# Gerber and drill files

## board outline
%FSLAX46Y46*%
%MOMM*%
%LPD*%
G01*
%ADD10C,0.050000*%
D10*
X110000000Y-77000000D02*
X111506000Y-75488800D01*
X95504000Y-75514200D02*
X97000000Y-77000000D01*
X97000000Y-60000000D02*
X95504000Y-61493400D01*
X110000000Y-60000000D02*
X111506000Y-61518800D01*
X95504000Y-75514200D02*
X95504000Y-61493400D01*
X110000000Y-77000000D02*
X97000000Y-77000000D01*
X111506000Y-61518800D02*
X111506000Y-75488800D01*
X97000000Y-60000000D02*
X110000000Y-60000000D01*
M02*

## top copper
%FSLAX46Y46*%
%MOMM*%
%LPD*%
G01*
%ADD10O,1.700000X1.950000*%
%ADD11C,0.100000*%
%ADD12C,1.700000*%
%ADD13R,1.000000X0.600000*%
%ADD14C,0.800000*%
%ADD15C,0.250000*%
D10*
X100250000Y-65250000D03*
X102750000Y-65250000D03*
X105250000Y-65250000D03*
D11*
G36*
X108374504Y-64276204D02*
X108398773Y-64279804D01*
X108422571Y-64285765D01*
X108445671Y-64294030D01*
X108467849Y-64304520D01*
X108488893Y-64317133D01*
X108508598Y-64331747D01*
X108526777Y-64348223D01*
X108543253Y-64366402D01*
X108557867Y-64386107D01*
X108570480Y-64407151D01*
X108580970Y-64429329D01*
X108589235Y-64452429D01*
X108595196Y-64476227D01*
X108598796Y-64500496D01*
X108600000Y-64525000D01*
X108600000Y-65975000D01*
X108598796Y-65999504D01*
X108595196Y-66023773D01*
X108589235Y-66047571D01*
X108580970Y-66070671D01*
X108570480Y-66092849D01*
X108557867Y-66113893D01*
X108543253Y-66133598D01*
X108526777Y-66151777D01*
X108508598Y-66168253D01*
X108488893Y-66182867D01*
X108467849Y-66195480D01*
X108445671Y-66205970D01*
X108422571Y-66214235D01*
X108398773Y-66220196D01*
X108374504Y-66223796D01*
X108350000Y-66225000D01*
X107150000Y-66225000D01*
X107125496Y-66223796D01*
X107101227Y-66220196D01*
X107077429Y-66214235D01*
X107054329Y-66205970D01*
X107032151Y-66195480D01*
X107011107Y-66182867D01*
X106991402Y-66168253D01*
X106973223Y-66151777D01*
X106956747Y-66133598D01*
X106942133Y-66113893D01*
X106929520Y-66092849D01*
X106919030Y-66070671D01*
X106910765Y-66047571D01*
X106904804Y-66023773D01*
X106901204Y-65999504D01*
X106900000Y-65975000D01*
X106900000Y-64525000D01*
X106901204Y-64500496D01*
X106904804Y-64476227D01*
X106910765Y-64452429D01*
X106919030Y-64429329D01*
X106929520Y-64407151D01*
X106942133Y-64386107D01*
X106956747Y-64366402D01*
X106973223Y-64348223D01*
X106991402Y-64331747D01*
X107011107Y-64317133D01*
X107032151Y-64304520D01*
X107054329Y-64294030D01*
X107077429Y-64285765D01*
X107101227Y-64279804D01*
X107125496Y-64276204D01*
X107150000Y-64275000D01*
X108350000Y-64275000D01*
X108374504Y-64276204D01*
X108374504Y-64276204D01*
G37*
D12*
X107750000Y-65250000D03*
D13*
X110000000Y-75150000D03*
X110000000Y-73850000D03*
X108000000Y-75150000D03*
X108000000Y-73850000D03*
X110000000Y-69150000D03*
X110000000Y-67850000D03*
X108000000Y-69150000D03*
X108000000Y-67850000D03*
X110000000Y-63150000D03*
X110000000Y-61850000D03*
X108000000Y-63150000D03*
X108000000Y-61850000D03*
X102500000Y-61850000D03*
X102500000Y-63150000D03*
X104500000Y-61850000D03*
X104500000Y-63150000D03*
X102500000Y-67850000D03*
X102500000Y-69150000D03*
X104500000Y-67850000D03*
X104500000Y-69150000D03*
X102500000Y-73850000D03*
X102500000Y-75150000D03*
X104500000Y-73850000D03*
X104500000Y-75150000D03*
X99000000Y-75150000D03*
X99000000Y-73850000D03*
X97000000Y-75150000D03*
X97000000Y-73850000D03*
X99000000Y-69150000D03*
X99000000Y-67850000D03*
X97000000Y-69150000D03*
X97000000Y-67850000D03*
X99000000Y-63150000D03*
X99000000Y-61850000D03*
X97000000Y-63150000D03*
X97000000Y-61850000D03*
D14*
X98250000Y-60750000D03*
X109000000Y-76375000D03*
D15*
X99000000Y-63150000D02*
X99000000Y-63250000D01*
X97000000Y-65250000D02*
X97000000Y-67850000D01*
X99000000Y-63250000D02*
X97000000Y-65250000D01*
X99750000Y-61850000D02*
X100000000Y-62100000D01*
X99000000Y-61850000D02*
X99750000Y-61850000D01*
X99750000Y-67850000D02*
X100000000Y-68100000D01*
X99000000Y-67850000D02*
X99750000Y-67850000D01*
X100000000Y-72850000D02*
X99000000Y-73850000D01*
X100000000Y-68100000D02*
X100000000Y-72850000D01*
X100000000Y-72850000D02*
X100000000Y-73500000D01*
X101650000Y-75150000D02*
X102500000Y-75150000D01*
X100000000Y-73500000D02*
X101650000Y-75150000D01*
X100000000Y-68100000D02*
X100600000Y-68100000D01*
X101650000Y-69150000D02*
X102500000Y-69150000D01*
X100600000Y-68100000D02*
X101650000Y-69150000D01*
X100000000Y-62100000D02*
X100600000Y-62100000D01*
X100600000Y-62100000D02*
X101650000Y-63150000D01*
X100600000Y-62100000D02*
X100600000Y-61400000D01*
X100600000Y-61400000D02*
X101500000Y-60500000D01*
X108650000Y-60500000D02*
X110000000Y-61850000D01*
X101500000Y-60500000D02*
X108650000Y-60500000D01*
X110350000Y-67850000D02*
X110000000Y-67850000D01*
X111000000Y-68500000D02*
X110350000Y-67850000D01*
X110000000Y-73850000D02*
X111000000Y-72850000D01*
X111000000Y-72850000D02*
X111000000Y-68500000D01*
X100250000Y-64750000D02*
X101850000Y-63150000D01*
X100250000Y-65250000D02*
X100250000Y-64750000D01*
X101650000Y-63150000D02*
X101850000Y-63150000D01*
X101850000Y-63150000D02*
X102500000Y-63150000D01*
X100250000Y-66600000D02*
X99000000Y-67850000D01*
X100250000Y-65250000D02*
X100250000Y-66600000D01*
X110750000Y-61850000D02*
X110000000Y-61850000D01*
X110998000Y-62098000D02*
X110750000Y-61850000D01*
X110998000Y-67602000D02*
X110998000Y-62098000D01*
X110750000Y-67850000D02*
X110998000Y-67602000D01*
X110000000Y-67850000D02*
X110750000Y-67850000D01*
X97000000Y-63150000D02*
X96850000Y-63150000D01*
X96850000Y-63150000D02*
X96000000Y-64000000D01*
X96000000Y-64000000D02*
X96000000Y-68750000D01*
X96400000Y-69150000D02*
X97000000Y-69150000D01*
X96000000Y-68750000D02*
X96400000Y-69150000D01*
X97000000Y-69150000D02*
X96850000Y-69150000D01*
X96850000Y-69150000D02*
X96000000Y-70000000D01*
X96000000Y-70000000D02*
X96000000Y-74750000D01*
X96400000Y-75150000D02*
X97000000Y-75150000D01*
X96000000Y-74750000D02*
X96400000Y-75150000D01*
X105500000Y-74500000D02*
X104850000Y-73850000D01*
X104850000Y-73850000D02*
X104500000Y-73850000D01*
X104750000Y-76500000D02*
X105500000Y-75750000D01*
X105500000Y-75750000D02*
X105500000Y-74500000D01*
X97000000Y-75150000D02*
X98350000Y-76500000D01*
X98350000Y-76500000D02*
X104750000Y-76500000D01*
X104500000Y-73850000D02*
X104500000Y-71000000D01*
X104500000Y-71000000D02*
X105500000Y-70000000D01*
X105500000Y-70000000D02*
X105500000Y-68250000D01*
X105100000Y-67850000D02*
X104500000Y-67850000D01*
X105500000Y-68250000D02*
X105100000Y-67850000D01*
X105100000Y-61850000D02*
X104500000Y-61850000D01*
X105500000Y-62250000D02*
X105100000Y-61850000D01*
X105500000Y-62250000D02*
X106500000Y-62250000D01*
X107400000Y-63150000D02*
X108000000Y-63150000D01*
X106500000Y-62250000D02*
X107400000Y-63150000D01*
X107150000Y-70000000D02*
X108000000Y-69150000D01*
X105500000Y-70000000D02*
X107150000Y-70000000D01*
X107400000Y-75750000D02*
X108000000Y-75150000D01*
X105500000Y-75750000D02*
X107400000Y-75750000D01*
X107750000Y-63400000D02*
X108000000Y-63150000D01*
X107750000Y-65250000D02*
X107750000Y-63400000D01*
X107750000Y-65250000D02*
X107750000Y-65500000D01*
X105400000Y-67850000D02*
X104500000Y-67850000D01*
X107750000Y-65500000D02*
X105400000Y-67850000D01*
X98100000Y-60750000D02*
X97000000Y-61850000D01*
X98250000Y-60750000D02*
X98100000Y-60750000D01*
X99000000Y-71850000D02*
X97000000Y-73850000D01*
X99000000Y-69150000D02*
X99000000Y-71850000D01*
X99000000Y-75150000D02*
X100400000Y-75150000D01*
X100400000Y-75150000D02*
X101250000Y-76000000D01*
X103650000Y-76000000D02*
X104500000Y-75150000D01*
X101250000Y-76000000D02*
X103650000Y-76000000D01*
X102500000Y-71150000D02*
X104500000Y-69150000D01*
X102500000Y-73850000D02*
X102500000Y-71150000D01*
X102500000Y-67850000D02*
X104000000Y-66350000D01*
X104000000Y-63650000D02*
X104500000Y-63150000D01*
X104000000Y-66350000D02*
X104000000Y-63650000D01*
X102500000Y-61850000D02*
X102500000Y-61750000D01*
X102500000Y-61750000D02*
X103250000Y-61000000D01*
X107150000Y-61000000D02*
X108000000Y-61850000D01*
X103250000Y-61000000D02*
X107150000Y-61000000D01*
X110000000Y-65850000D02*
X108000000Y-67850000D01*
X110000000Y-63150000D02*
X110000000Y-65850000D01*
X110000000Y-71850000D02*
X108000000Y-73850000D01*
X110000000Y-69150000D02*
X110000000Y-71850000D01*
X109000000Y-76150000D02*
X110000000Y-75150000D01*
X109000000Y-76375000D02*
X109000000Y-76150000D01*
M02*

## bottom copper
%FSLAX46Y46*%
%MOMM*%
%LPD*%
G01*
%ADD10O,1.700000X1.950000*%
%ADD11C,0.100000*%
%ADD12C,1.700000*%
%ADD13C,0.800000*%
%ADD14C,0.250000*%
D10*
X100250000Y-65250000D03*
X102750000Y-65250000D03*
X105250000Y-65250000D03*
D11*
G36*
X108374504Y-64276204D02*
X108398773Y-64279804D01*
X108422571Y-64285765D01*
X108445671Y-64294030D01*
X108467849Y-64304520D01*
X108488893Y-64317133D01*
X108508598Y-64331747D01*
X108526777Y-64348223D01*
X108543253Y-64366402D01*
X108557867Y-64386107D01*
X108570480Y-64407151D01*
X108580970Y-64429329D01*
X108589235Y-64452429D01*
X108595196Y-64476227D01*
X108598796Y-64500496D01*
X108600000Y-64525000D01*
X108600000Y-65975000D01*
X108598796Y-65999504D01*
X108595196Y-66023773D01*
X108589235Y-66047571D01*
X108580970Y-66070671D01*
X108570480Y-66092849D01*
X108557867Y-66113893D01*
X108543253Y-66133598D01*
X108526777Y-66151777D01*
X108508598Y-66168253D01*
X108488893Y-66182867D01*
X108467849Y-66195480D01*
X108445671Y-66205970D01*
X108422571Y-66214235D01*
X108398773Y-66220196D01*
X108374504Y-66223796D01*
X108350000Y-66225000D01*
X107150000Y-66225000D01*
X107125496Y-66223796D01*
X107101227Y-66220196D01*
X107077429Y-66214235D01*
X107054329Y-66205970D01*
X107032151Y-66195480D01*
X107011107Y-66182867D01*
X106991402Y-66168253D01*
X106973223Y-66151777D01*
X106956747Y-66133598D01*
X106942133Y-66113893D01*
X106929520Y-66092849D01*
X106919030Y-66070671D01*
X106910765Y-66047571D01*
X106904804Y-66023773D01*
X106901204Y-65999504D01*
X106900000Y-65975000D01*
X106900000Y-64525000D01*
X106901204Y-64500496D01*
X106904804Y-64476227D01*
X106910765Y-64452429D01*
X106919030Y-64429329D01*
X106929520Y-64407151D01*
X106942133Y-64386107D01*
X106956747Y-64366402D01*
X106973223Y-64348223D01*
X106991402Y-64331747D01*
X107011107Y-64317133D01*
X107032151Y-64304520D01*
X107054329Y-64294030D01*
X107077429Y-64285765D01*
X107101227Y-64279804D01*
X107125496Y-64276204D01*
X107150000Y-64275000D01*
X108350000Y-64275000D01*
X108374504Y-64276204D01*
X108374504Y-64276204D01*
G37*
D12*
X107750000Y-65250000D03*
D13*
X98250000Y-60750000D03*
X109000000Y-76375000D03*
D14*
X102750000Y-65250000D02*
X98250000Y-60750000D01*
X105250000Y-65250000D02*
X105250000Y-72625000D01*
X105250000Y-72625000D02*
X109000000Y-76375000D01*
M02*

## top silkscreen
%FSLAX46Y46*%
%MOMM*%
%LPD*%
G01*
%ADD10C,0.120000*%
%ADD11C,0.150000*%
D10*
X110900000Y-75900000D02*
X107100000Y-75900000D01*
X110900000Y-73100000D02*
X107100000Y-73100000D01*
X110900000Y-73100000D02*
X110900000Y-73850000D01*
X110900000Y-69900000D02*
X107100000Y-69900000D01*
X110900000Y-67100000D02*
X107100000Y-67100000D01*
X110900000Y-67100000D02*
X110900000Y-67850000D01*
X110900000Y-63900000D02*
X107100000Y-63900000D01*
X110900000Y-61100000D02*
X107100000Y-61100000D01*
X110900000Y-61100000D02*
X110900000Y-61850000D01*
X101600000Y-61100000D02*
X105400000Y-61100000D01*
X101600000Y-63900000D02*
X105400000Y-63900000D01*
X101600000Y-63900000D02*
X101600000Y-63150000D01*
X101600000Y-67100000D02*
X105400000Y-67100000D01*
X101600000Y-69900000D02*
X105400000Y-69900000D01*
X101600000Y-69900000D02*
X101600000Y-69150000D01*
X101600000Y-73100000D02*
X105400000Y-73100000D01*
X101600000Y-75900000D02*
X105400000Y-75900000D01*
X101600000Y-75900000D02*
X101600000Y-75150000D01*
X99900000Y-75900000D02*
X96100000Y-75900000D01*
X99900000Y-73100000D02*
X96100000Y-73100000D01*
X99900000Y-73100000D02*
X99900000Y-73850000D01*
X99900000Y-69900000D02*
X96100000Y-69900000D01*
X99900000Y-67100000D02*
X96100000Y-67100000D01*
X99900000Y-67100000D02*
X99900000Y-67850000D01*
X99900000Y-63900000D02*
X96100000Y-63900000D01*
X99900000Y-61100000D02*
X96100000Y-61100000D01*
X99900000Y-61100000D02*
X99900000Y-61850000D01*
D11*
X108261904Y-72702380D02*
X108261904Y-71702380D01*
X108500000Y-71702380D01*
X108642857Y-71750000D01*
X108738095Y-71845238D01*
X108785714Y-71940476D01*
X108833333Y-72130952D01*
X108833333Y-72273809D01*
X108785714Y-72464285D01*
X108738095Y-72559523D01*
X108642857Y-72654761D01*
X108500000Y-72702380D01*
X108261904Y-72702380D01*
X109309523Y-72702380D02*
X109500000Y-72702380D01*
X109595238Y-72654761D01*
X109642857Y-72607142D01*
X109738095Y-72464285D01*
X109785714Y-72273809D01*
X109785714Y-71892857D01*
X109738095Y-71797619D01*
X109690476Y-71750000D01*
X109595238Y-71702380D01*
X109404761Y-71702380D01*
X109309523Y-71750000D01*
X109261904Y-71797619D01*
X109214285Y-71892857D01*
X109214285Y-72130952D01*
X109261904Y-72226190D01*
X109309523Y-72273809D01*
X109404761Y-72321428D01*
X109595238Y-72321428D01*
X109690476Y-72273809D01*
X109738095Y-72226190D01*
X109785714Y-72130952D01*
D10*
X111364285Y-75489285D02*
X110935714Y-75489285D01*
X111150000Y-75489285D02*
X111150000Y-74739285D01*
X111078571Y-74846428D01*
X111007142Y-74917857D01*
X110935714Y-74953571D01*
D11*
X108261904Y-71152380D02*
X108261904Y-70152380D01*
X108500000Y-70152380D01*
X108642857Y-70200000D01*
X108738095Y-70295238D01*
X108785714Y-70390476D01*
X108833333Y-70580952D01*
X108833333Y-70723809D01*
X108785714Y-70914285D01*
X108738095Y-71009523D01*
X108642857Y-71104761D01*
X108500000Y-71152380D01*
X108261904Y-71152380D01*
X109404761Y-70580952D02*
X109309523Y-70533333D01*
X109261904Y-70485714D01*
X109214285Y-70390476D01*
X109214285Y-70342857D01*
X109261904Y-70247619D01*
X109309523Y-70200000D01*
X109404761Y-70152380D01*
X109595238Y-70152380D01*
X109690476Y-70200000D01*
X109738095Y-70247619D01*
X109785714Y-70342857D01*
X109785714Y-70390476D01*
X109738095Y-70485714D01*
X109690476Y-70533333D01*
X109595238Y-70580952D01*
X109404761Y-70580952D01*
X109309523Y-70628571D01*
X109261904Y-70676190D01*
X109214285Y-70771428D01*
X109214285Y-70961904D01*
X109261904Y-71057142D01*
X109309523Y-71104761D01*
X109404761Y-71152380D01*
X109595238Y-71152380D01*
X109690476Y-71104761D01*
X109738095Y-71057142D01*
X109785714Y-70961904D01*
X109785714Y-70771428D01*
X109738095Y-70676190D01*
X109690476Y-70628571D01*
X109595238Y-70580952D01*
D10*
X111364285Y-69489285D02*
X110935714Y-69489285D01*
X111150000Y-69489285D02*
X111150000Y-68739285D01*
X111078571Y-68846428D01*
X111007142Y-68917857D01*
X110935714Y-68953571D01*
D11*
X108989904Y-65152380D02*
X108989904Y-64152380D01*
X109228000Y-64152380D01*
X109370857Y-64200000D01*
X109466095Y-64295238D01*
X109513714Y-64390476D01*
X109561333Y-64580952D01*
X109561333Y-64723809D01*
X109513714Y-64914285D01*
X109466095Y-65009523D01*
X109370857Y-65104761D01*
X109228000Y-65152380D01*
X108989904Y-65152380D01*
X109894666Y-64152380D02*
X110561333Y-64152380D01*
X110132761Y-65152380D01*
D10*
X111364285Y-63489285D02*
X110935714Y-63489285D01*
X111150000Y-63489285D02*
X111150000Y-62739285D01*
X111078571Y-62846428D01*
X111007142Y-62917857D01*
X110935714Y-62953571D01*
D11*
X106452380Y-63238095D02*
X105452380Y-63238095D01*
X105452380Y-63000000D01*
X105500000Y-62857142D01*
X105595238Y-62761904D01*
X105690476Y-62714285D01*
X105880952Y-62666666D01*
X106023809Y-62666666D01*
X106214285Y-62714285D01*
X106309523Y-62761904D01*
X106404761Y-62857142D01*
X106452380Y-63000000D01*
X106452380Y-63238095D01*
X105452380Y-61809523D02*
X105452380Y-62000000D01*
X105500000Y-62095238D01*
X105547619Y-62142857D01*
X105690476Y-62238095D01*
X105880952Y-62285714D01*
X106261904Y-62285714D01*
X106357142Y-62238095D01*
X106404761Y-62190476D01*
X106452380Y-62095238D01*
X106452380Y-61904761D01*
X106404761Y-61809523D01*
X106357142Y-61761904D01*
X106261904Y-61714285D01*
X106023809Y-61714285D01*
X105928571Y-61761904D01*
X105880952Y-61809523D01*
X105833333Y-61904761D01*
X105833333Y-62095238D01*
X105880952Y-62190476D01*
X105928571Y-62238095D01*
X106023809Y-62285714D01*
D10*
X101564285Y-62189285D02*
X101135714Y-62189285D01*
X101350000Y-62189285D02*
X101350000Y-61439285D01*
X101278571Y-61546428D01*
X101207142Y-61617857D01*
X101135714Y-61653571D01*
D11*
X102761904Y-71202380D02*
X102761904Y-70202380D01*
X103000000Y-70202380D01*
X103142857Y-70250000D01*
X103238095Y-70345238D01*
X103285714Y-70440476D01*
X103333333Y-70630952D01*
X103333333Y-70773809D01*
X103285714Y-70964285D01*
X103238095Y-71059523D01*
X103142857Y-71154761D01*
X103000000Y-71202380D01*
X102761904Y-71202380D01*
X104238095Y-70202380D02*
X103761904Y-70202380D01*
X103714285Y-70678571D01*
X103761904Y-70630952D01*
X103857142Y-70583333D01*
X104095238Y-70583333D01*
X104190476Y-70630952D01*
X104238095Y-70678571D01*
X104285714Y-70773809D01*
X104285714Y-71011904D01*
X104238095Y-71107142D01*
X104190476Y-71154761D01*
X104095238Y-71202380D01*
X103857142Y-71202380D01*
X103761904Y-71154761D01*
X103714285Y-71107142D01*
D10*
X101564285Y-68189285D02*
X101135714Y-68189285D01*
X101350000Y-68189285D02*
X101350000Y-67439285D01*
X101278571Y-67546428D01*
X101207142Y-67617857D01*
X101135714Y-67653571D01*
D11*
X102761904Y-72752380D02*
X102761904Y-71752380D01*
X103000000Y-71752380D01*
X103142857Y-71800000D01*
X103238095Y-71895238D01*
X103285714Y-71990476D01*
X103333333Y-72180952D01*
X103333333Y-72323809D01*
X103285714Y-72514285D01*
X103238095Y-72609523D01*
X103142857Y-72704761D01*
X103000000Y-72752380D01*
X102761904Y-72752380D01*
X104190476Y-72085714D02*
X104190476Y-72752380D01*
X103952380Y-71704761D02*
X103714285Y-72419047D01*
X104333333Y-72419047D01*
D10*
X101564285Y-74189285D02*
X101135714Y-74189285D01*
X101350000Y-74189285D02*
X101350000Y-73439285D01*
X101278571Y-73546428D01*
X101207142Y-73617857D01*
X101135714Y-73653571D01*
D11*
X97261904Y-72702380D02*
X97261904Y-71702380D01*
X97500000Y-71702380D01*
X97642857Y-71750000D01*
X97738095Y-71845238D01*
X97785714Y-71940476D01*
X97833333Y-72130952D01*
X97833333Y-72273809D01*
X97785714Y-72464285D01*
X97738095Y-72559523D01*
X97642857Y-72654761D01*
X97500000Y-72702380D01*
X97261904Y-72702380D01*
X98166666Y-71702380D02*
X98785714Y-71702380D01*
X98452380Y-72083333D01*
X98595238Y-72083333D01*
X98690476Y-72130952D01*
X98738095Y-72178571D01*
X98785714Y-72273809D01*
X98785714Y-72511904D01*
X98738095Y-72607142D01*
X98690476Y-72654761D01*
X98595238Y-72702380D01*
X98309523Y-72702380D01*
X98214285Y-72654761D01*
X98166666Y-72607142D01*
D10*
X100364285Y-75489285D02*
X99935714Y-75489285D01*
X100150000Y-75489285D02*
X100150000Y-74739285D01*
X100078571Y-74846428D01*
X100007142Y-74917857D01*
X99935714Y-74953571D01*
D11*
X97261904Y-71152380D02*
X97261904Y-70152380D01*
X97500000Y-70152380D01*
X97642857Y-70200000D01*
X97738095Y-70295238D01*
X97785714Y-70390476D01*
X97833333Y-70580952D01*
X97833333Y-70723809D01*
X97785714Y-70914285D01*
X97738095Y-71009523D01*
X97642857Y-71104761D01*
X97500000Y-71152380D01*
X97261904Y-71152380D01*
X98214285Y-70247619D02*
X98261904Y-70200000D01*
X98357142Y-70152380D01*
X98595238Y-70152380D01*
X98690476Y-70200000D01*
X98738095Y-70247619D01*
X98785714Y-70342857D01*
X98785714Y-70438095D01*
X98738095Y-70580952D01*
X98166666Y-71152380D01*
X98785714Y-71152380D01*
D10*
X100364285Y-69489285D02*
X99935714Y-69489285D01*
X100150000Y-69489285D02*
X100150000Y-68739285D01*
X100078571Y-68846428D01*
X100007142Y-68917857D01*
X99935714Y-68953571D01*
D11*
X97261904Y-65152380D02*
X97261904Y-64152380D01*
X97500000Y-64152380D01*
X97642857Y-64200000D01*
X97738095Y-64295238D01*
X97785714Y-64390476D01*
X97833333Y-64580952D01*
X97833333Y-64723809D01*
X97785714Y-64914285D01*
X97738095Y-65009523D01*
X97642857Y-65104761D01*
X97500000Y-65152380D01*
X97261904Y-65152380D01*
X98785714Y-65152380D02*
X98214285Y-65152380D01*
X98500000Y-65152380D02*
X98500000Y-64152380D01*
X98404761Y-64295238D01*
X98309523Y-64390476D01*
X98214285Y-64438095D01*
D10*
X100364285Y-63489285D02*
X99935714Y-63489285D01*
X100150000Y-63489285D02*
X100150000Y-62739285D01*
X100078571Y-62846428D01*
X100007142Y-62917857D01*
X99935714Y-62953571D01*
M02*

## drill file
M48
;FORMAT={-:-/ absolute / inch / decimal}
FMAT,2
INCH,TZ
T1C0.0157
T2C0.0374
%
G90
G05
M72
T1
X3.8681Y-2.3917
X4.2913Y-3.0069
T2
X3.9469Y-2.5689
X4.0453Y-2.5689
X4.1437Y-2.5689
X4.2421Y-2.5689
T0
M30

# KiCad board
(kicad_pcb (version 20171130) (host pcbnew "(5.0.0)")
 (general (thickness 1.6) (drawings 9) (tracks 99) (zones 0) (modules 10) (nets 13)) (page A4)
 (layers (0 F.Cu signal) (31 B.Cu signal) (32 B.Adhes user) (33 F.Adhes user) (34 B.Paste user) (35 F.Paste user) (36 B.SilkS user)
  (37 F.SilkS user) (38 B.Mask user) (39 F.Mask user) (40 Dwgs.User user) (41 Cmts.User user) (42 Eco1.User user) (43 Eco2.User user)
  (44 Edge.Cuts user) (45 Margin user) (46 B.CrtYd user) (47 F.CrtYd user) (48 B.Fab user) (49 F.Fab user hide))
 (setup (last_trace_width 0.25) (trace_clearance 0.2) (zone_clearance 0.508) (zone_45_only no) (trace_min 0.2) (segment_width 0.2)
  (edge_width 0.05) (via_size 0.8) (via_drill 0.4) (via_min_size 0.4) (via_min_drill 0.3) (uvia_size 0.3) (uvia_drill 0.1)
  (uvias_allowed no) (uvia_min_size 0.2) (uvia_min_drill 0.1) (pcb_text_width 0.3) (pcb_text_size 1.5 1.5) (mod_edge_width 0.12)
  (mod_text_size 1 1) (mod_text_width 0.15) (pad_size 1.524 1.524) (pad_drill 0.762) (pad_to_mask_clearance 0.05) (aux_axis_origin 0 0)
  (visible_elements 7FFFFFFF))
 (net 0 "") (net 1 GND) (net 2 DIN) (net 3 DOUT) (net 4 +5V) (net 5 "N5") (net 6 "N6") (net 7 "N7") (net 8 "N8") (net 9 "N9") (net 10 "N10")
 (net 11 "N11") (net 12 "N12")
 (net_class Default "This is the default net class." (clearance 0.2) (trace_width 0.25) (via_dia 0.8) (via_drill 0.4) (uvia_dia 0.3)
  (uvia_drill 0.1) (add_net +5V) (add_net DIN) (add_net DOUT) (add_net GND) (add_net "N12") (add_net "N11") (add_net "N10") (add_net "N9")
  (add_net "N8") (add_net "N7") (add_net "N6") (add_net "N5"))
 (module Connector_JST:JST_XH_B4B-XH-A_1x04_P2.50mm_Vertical (layer B.Cu) (at 107.75 65.25 180)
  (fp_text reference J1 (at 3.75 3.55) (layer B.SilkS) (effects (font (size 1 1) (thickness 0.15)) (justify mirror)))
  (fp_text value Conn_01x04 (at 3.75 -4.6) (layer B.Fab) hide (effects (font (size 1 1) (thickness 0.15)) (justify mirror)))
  (pad 4 thru_hole oval (at 7.5 0 180) (size 1.7 1.95) (drill 0.95) (layers *.Cu *.Mask) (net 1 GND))
  (pad 3 thru_hole oval (at 5 0 180) (size 1.7 1.95) (drill 0.95) (layers *.Cu *.Mask) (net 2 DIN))
  (pad 2 thru_hole oval (at 2.5 0 180) (size 1.7 1.95) (drill 0.95) (layers *.Cu *.Mask) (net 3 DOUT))
  (pad 1 thru_hole roundrect (at 0 0 180) (size 1.7 1.95) (drill 0.95) (layers *.Cu *.Mask) (roundrect_rratio 0.147059) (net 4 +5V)))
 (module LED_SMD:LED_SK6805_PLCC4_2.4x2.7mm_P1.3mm (layer F.Cu) (at 109 74.5 180)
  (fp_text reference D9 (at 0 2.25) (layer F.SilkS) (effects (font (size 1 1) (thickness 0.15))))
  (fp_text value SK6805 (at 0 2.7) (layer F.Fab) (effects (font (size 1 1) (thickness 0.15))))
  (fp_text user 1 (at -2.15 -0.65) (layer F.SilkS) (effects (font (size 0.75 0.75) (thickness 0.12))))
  (fp_line (start -1.9 -1.4) (end 1.9 -1.4) (layer F.SilkS) (width 0.12))
  (fp_line (start -1.9 1.4) (end 1.9 1.4) (layer F.SilkS) (width 0.12))
  (fp_line (start -1.9 1.4) (end -1.9 0.65) (layer F.SilkS) (width 0.12))
  (pad 1 smd rect (at -1 -0.65 180) (size 1 0.6) (layers F.Cu F.Paste F.Mask) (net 3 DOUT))
  (pad 2 smd rect (at -1 0.65 180) (size 1 0.6) (layers F.Cu F.Paste F.Mask) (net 1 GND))
  (pad 4 smd rect (at 1 -0.65 180) (size 1 0.6) (layers F.Cu F.Paste F.Mask) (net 4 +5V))
  (pad 3 smd rect (at 1 0.65 180) (size 1 0.6) (layers F.Cu F.Paste F.Mask) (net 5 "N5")))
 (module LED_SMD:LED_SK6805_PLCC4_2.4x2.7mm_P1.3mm (layer F.Cu) (at 109 68.5 180)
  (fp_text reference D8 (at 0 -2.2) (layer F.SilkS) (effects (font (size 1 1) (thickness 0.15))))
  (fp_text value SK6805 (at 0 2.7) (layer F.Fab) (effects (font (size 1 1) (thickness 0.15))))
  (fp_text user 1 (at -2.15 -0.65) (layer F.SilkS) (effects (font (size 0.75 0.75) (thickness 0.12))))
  (fp_line (start -1.9 -1.4) (end 1.9 -1.4) (layer F.SilkS) (width 0.12))
  (fp_line (start -1.9 1.4) (end 1.9 1.4) (layer F.SilkS) (width 0.12))
  (fp_line (start -1.9 1.4) (end -1.9 0.65) (layer F.SilkS) (width 0.12))
  (pad 1 smd rect (at -1 -0.65 180) (size 1 0.6) (layers F.Cu F.Paste F.Mask) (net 5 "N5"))
  (pad 2 smd rect (at -1 0.65 180) (size 1 0.6) (layers F.Cu F.Paste F.Mask) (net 1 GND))
  (pad 4 smd rect (at 1 -0.65 180) (size 1 0.6) (layers F.Cu F.Paste F.Mask) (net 4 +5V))
  (pad 3 smd rect (at 1 0.65 180) (size 1 0.6) (layers F.Cu F.Paste F.Mask) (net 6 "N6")))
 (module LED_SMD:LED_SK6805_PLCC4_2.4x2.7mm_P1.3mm (layer F.Cu) (at 109 62.5 180)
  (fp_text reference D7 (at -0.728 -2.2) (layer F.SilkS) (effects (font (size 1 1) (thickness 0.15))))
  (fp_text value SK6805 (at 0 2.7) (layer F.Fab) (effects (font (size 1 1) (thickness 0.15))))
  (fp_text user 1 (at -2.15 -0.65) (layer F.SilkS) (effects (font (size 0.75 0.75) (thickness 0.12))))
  (fp_line (start -1.9 -1.4) (end 1.9 -1.4) (layer F.SilkS) (width 0.12))
  (fp_line (start -1.9 1.4) (end 1.9 1.4) (layer F.SilkS) (width 0.12))
  (fp_line (start -1.9 1.4) (end -1.9 0.65) (layer F.SilkS) (width 0.12))
  (pad 1 smd rect (at -1 -0.65 180) (size 1 0.6) (layers F.Cu F.Paste F.Mask) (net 6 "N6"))
  (pad 2 smd rect (at -1 0.65 180) (size 1 0.6) (layers F.Cu F.Paste F.Mask) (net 1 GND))
  (pad 4 smd rect (at 1 -0.65 180) (size 1 0.6) (layers F.Cu F.Paste F.Mask) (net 4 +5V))
  (pad 3 smd rect (at 1 0.65 180) (size 1 0.6) (layers F.Cu F.Paste F.Mask) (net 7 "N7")))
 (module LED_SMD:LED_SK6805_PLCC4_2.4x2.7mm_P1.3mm (layer F.Cu) (at 103.5 62.5)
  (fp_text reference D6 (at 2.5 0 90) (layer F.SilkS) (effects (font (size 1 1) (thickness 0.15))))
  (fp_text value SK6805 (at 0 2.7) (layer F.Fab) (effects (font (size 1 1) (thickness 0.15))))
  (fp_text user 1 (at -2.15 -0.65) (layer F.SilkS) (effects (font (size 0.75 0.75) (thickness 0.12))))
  (fp_line (start -1.9 -1.4) (end 1.9 -1.4) (layer F.SilkS) (width 0.12))
  (fp_line (start -1.9 1.4) (end 1.9 1.4) (layer F.SilkS) (width 0.12))
  (fp_line (start -1.9 1.4) (end -1.9 0.65) (layer F.SilkS) (width 0.12))
  (pad 1 smd rect (at -1 -0.65) (size 1 0.6) (layers F.Cu F.Paste F.Mask) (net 7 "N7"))
  (pad 2 smd rect (at -1 0.65) (size 1 0.6) (layers F.Cu F.Paste F.Mask) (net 1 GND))
  (pad 4 smd rect (at 1 -0.65) (size 1 0.6) (layers F.Cu F.Paste F.Mask) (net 4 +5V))
  (pad 3 smd rect (at 1 0.65) (size 1 0.6) (layers F.Cu F.Paste F.Mask) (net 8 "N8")))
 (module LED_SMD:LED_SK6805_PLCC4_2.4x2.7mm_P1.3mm (layer F.Cu) (at 103.5 68.5)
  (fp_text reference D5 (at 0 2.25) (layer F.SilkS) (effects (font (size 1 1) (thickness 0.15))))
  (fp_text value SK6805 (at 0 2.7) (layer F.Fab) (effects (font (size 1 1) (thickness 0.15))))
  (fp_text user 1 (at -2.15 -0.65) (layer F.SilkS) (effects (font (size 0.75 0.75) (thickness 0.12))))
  (fp_line (start -1.9 -1.4) (end 1.9 -1.4) (layer F.SilkS) (width 0.12))
  (fp_line (start -1.9 1.4) (end 1.9 1.4) (layer F.SilkS) (width 0.12))
  (fp_line (start -1.9 1.4) (end -1.9 0.65) (layer F.SilkS) (width 0.12))
  (pad 1 smd rect (at -1 -0.65) (size 1 0.6) (layers F.Cu F.Paste F.Mask) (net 8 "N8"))
  (pad 2 smd rect (at -1 0.65) (size 1 0.6) (layers F.Cu F.Paste F.Mask) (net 1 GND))
  (pad 4 smd rect (at 1 -0.65) (size 1 0.6) (layers F.Cu F.Paste F.Mask) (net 4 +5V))
  (pad 3 smd rect (at 1 0.65) (size 1 0.6) (layers F.Cu F.Paste F.Mask) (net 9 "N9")))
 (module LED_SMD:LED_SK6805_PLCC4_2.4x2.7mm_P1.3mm (layer F.Cu) (at 103.5 74.5)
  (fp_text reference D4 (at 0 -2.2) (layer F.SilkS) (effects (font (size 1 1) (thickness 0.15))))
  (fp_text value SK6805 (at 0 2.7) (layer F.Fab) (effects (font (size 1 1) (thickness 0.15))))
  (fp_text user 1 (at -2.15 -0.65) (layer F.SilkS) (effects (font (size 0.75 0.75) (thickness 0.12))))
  (fp_line (start -1.9 -1.4) (end 1.9 -1.4) (layer F.SilkS) (width 0.12))
  (fp_line (start -1.9 1.4) (end 1.9 1.4) (layer F.SilkS) (width 0.12))
  (fp_line (start -1.9 1.4) (end -1.9 0.65) (layer F.SilkS) (width 0.12))
  (pad 1 smd rect (at -1 -0.65) (size 1 0.6) (layers F.Cu F.Paste F.Mask) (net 9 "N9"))
  (pad 2 smd rect (at -1 0.65) (size 1 0.6) (layers F.Cu F.Paste F.Mask) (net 1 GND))
  (pad 4 smd rect (at 1 -0.65) (size 1 0.6) (layers F.Cu F.Paste F.Mask) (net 4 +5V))
  (pad 3 smd rect (at 1 0.65) (size 1 0.6) (layers F.Cu F.Paste F.Mask) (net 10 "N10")))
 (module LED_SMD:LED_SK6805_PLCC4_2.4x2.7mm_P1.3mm (layer F.Cu) (at 98 74.5 180)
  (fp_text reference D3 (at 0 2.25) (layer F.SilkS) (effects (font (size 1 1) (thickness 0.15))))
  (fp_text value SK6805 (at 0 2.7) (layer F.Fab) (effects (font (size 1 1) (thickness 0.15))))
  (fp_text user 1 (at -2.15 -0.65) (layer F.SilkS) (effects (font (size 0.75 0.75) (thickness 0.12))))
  (fp_line (start -1.9 -1.4) (end 1.9 -1.4) (layer F.SilkS) (width 0.12))
  (fp_line (start -1.9 1.4) (end 1.9 1.4) (layer F.SilkS) (width 0.12))
  (fp_line (start -1.9 1.4) (end -1.9 0.65) (layer F.SilkS) (width 0.12))
  (pad 1 smd rect (at -1 -0.65 180) (size 1 0.6) (layers F.Cu F.Paste F.Mask) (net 10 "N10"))
  (pad 2 smd rect (at -1 0.65 180) (size 1 0.6) (layers F.Cu F.Paste F.Mask) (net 1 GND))
  (pad 4 smd rect (at 1 -0.65 180) (size 1 0.6) (layers F.Cu F.Paste F.Mask) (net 4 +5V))
  (pad 3 smd rect (at 1 0.65 180) (size 1 0.6) (layers F.Cu F.Paste F.Mask) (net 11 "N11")))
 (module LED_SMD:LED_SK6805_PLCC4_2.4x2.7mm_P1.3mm (layer F.Cu) (at 98 68.5 180)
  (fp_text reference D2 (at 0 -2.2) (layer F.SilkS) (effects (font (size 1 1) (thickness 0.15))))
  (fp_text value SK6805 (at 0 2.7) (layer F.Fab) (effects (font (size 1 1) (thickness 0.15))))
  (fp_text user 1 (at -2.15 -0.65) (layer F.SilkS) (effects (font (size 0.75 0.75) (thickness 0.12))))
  (fp_line (start -1.9 -1.4) (end 1.9 -1.4) (layer F.SilkS) (width 0.12))
  (fp_line (start -1.9 1.4) (end 1.9 1.4) (layer F.SilkS) (width 0.12))
  (fp_line (start -1.9 1.4) (end -1.9 0.65) (layer F.SilkS) (width 0.12))
  (pad 1 smd rect (at -1 -0.65 180) (size 1 0.6) (layers F.Cu F.Paste F.Mask) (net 11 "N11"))
  (pad 2 smd rect (at -1 0.65 180) (size 1 0.6) (layers F.Cu F.Paste F.Mask) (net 1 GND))
  (pad 4 smd rect (at 1 -0.65 180) (size 1 0.6) (layers F.Cu F.Paste F.Mask) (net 4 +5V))
  (pad 3 smd rect (at 1 0.65 180) (size 1 0.6) (layers F.Cu F.Paste F.Mask) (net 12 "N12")))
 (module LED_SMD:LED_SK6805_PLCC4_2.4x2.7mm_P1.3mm (layer F.Cu) (at 98 62.5 180)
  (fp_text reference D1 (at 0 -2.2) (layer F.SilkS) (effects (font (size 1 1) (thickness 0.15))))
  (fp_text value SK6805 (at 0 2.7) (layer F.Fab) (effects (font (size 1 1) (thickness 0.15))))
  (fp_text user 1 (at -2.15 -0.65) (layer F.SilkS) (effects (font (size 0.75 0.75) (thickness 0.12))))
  (fp_line (start -1.9 -1.4) (end 1.9 -1.4) (layer F.SilkS) (width 0.12))
  (fp_line (start -1.9 1.4) (end 1.9 1.4) (layer F.SilkS) (width 0.12))
  (fp_line (start -1.9 1.4) (end -1.9 0.65) (layer F.SilkS) (width 0.12))
  (pad 1 smd rect (at -1 -0.65 180) (size 1 0.6) (layers F.Cu F.Paste F.Mask) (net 12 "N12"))
  (pad 2 smd rect (at -1 0.65 180) (size 1 0.6) (layers F.Cu F.Paste F.Mask) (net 1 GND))
  (pad 4 smd rect (at 1 -0.65 180) (size 1 0.6) (layers F.Cu F.Paste F.Mask) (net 4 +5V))
  (pad 3 smd rect (at 1 0.65 180) (size 1 0.6) (layers F.Cu F.Paste F.Mask) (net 2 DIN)))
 (gr_line (start 110 77) (end 111.506 75.4888) (layer Edge.Cuts) (width 0.05))
 (gr_line (start 95.504 75.5142) (end 97 77) (layer Edge.Cuts) (width 0.05))
 (gr_line (start 97 60) (end 95.504 61.4934) (layer Edge.Cuts) (width 0.05))
 (gr_line (start 110 60) (end 111.506 61.5188) (layer Edge.Cuts) (width 0.05))
 (gr_line (start 95.504 75.5142) (end 95.504 61.4934) (layer Edge.Cuts) (width 0.05))
 (gr_line (start 110 77) (end 97 77) (layer Edge.Cuts) (width 0.05))
 (gr_line (start 111.506 61.5188) (end 111.506 75.4888) (layer Edge.Cuts) (width 0.05))
 (gr_line (start 97 60) (end 110 60) (layer Edge.Cuts) (width 0.05))
 (segment (start 99 63.15) (end 99 63.25) (width 0.25) (layer F.Cu) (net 12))
 (segment (start 97 65.25) (end 97 67.85) (width 0.25) (layer F.Cu) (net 12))
 (segment (start 99 63.25) (end 97 65.25) (width 0.25) (layer F.Cu) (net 12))
 (segment (start 99.75 61.85) (end 100 62.1) (width 0.25) (layer F.Cu) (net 1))
 (segment (start 99 61.85) (end 99.75 61.85) (width 0.25) (layer F.Cu) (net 1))
 (segment (start 99.75 67.85) (end 100 68.1) (width 0.25) (layer F.Cu) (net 1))
 (segment (start 99 67.85) (end 99.75 67.85) (width 0.25) (layer F.Cu) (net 1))
 (segment (start 100 72.85) (end 99 73.85) (width 0.25) (layer F.Cu) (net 1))
 (segment (start 100 68.1) (end 100 72.85) (width 0.25) (layer F.Cu) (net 1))
 (segment (start 100 72.85) (end 100 73.5) (width 0.25) (layer F.Cu) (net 1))
 (segment (start 101.65 75.15) (end 102.5 75.15) (width 0.25) (layer F.Cu) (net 1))
 (segment (start 100 73.5) (end 101.65 75.15) (width 0.25) (layer F.Cu) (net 1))
 (segment (start 100 68.1) (end 100.6 68.1) (width 0.25) (layer F.Cu) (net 1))
 (segment (start 101.65 69.15) (end 102.5 69.15) (width 0.25) (layer F.Cu) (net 1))
 (segment (start 100.6 68.1) (end 101.65 69.15) (width 0.25) (layer F.Cu) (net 1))
 (segment (start 100 62.1) (end 100.6 62.1) (width 0.25) (layer F.Cu) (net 1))
 (segment (start 100.6 62.1) (end 101.65 63.15) (width 0.25) (layer F.Cu) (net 1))
 (segment (start 100.6 62.1) (end 100.6 61.4) (width 0.25) (layer F.Cu) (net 1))
 (segment (start 100.6 61.4) (end 101.5 60.5) (width 0.25) (layer F.Cu) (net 1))
 (segment (start 108.65 60.5) (end 110 61.85) (width 0.25) (layer F.Cu) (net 1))
 (segment (start 101.5 60.5) (end 108.65 60.5) (width 0.25) (layer F.Cu) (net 1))
 (segment (start 110.35 67.85) (end 110 67.85) (width 0.25) (layer F.Cu) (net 1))
 (segment (start 111 68.5) (end 110.35 67.85) (width 0.25) (layer F.Cu) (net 1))
 (segment (start 110 73.85) (end 111 72.85) (width 0.25) (layer F.Cu) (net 1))
 (segment (start 111 72.85) (end 111 68.5) (width 0.25) (layer F.Cu) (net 1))
 (segment (start 100.25 64.75) (end 101.85 63.15) (width 0.25) (layer F.Cu) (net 1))
 (segment (start 100.25 65.25) (end 100.25 64.75) (width 0.25) (layer F.Cu) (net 1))
 (segment (start 101.65 63.15) (end 101.85 63.15) (width 0.25) (layer F.Cu) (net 1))
 (segment (start 101.85 63.15) (end 102.5 63.15) (width 0.25) (layer F.Cu) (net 1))
 (segment (start 100.25 66.6) (end 99 67.85) (width 0.25) (layer F.Cu) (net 1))
 (segment (start 100.25 65.25) (end 100.25 66.6) (width 0.25) (layer F.Cu) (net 1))
 (segment (start 110.75 61.85) (end 110 61.85) (width 0.25) (layer F.Cu) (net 1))
 (segment (start 110.998 62.098) (end 110.75 61.85) (width 0.25) (layer F.Cu) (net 1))
 (segment (start 110.998 67.602) (end 110.998 62.098) (width 0.25) (layer F.Cu) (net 1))
 (segment (start 110.75 67.85) (end 110.998 67.602) (width 0.25) (layer F.Cu) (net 1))
 (segment (start 110 67.85) (end 110.75 67.85) (width 0.25) (layer F.Cu) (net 1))
 (segment (start 97 63.15) (end 96.85 63.15) (width 0.25) (layer F.Cu) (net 4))
 (segment (start 96.85 63.15) (end 96 64) (width 0.25) (layer F.Cu) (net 4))
 (segment (start 96 64) (end 96 68.75) (width 0.25) (layer F.Cu) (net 4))
 (segment (start 96.4 69.15) (end 97 69.15) (width 0.25) (layer F.Cu) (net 4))
 (segment (start 96 68.75) (end 96.4 69.15) (width 0.25) (layer F.Cu) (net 4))
 (segment (start 97 69.15) (end 96.85 69.15) (width 0.25) (layer F.Cu) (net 4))
 (segment (start 96.85 69.15) (end 96 70) (width 0.25) (layer F.Cu) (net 4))
 (segment (start 96 70) (end 96 74.75) (width 0.25) (layer F.Cu) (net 4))
 (segment (start 96.4 75.15) (end 97 75.15) (width 0.25) (layer F.Cu) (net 4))
 (segment (start 96 74.75) (end 96.4 75.15) (width 0.25) (layer F.Cu) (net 4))
 (segment (start 105.5 74.5) (end 104.85 73.85) (width 0.25) (layer F.Cu) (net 4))
 (segment (start 104.85 73.85) (end 104.5 73.85) (width 0.25) (layer F.Cu) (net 4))
 (segment (start 104.75 76.5) (end 105.5 75.75) (width 0.25) (layer F.Cu) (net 4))
 (segment (start 105.5 75.75) (end 105.5 74.5) (width 0.25) (layer F.Cu) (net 4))
 (segment (start 97 75.15) (end 98.35 76.5) (width 0.25) (layer F.Cu) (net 4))
 (segment (start 98.35 76.5) (end 104.75 76.5) (width 0.25) (layer F.Cu) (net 4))
 (segment (start 104.5 73.85) (end 104.5 71) (width 0.25) (layer F.Cu) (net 4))
 (segment (start 104.5 71) (end 105.5 70) (width 0.25) (layer F.Cu) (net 4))
 (segment (start 105.5 70) (end 105.5 68.25) (width 0.25) (layer F.Cu) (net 4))
 (segment (start 105.1 67.85) (end 104.5 67.85) (width 0.25) (layer F.Cu) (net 4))
 (segment (start 105.5 68.25) (end 105.1 67.85) (width 0.25) (layer F.Cu) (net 4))
 (segment (start 105.1 61.85) (end 104.5 61.85) (width 0.25) (layer F.Cu) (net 4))
 (segment (start 105.5 62.25) (end 105.1 61.85) (width 0.25) (layer F.Cu) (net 4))
 (segment (start 105.5 62.25) (end 106.5 62.25) (width 0.25) (layer F.Cu) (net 4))
 (segment (start 107.4 63.15) (end 108 63.15) (width 0.25) (layer F.Cu) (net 4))
 (segment (start 106.5 62.25) (end 107.4 63.15) (width 0.25) (layer F.Cu) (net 4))
 (segment (start 107.15 70) (end 108 69.15) (width 0.25) (layer F.Cu) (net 4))
 (segment (start 105.5 70) (end 107.15 70) (width 0.25) (layer F.Cu) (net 4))
 (segment (start 107.4 75.75) (end 108 75.15) (width 0.25) (layer F.Cu) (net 4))
 (segment (start 105.5 75.75) (end 107.4 75.75) (width 0.25) (layer F.Cu) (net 4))
 (segment (start 107.75 63.4) (end 108 63.15) (width 0.25) (layer F.Cu) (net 4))
 (segment (start 107.75 65.25) (end 107.75 63.4) (width 0.25) (layer F.Cu) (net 4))
 (segment (start 107.75 65.25) (end 107.75 65.5) (width 0.25) (layer F.Cu) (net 4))
 (segment (start 105.4 67.85) (end 104.5 67.85) (width 0.25) (layer F.Cu) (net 4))
 (segment (start 107.75 65.5) (end 105.4 67.85) (width 0.25) (layer F.Cu) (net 4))
 (via (at 98.25 60.75) (size 0.8) (drill 0.4) (layers F.Cu B.Cu) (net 2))
 (segment (start 102.75 65.25) (end 98.25 60.75) (width 0.25) (layer B.Cu) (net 2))
 (segment (start 98.1 60.75) (end 97 61.85) (width 0.25) (layer F.Cu) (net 2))
 (segment (start 98.25 60.75) (end 98.1 60.75) (width 0.25) (layer F.Cu) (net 2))
 (segment (start 99 71.85) (end 97 73.85) (width 0.25) (layer F.Cu) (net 11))
 (segment (start 99 69.15) (end 99 71.85) (width 0.25) (layer F.Cu) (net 11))
 (segment (start 99 75.15) (end 100.4 75.15) (width 0.25) (layer F.Cu) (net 10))
 (segment (start 100.4 75.15) (end 101.25 76) (width 0.25) (layer F.Cu) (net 10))
 (segment (start 103.65 76) (end 104.5 75.15) (width 0.25) (layer F.Cu) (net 10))
 (segment (start 101.25 76) (end 103.65 76) (width 0.25) (layer F.Cu) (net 10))
 (segment (start 102.5 71.15) (end 104.5 69.15) (width 0.25) (layer F.Cu) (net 9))
 (segment (start 102.5 73.85) (end 102.5 71.15) (width 0.25) (layer F.Cu) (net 9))
 (segment (start 102.5 67.85) (end 104 66.35) (width 0.25) (layer F.Cu) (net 8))
 (segment (start 104 63.65) (end 104.5 63.15) (width 0.25) (layer F.Cu) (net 8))
 (segment (start 104 66.35) (end 104 63.65) (width 0.25) (layer F.Cu) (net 8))
 (segment (start 102.5 61.85) (end 102.5 61.75) (width 0.25) (layer F.Cu) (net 7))
 (segment (start 102.5 61.75) (end 103.25 61) (width 0.25) (layer F.Cu) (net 7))
 (segment (start 107.15 61) (end 108 61.85) (width 0.25) (layer F.Cu) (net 7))
 (segment (start 103.25 61) (end 107.15 61) (width 0.25) (layer F.Cu) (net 7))
 (segment (start 110 65.85) (end 108 67.85) (width 0.25) (layer F.Cu) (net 6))
 (segment (start 110 63.15) (end 110 65.85) (width 0.25) (layer F.Cu) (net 6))
 (segment (start 110 71.85) (end 108 73.85) (width 0.25) (layer F.Cu) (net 5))
 (segment (start 110 69.15) (end 110 71.85) (width 0.25) (layer F.Cu) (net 5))
 (via (at 109 76.375) (size 0.8) (drill 0.4) (layers F.Cu B.Cu) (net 3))
 (segment (start 105.25 65.25) (end 105.25 72.625) (width 0.25) (layer B.Cu) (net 3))
 (segment (start 105.25 72.625) (end 109 76.375) (width 0.25) (layer B.Cu) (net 3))
 (segment (start 109 76.15) (end 110 75.15) (width 0.25) (layer F.Cu) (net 3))
 (segment (start 109 76.375) (end 109 76.15) (width 0.25) (layer F.Cu) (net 3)))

